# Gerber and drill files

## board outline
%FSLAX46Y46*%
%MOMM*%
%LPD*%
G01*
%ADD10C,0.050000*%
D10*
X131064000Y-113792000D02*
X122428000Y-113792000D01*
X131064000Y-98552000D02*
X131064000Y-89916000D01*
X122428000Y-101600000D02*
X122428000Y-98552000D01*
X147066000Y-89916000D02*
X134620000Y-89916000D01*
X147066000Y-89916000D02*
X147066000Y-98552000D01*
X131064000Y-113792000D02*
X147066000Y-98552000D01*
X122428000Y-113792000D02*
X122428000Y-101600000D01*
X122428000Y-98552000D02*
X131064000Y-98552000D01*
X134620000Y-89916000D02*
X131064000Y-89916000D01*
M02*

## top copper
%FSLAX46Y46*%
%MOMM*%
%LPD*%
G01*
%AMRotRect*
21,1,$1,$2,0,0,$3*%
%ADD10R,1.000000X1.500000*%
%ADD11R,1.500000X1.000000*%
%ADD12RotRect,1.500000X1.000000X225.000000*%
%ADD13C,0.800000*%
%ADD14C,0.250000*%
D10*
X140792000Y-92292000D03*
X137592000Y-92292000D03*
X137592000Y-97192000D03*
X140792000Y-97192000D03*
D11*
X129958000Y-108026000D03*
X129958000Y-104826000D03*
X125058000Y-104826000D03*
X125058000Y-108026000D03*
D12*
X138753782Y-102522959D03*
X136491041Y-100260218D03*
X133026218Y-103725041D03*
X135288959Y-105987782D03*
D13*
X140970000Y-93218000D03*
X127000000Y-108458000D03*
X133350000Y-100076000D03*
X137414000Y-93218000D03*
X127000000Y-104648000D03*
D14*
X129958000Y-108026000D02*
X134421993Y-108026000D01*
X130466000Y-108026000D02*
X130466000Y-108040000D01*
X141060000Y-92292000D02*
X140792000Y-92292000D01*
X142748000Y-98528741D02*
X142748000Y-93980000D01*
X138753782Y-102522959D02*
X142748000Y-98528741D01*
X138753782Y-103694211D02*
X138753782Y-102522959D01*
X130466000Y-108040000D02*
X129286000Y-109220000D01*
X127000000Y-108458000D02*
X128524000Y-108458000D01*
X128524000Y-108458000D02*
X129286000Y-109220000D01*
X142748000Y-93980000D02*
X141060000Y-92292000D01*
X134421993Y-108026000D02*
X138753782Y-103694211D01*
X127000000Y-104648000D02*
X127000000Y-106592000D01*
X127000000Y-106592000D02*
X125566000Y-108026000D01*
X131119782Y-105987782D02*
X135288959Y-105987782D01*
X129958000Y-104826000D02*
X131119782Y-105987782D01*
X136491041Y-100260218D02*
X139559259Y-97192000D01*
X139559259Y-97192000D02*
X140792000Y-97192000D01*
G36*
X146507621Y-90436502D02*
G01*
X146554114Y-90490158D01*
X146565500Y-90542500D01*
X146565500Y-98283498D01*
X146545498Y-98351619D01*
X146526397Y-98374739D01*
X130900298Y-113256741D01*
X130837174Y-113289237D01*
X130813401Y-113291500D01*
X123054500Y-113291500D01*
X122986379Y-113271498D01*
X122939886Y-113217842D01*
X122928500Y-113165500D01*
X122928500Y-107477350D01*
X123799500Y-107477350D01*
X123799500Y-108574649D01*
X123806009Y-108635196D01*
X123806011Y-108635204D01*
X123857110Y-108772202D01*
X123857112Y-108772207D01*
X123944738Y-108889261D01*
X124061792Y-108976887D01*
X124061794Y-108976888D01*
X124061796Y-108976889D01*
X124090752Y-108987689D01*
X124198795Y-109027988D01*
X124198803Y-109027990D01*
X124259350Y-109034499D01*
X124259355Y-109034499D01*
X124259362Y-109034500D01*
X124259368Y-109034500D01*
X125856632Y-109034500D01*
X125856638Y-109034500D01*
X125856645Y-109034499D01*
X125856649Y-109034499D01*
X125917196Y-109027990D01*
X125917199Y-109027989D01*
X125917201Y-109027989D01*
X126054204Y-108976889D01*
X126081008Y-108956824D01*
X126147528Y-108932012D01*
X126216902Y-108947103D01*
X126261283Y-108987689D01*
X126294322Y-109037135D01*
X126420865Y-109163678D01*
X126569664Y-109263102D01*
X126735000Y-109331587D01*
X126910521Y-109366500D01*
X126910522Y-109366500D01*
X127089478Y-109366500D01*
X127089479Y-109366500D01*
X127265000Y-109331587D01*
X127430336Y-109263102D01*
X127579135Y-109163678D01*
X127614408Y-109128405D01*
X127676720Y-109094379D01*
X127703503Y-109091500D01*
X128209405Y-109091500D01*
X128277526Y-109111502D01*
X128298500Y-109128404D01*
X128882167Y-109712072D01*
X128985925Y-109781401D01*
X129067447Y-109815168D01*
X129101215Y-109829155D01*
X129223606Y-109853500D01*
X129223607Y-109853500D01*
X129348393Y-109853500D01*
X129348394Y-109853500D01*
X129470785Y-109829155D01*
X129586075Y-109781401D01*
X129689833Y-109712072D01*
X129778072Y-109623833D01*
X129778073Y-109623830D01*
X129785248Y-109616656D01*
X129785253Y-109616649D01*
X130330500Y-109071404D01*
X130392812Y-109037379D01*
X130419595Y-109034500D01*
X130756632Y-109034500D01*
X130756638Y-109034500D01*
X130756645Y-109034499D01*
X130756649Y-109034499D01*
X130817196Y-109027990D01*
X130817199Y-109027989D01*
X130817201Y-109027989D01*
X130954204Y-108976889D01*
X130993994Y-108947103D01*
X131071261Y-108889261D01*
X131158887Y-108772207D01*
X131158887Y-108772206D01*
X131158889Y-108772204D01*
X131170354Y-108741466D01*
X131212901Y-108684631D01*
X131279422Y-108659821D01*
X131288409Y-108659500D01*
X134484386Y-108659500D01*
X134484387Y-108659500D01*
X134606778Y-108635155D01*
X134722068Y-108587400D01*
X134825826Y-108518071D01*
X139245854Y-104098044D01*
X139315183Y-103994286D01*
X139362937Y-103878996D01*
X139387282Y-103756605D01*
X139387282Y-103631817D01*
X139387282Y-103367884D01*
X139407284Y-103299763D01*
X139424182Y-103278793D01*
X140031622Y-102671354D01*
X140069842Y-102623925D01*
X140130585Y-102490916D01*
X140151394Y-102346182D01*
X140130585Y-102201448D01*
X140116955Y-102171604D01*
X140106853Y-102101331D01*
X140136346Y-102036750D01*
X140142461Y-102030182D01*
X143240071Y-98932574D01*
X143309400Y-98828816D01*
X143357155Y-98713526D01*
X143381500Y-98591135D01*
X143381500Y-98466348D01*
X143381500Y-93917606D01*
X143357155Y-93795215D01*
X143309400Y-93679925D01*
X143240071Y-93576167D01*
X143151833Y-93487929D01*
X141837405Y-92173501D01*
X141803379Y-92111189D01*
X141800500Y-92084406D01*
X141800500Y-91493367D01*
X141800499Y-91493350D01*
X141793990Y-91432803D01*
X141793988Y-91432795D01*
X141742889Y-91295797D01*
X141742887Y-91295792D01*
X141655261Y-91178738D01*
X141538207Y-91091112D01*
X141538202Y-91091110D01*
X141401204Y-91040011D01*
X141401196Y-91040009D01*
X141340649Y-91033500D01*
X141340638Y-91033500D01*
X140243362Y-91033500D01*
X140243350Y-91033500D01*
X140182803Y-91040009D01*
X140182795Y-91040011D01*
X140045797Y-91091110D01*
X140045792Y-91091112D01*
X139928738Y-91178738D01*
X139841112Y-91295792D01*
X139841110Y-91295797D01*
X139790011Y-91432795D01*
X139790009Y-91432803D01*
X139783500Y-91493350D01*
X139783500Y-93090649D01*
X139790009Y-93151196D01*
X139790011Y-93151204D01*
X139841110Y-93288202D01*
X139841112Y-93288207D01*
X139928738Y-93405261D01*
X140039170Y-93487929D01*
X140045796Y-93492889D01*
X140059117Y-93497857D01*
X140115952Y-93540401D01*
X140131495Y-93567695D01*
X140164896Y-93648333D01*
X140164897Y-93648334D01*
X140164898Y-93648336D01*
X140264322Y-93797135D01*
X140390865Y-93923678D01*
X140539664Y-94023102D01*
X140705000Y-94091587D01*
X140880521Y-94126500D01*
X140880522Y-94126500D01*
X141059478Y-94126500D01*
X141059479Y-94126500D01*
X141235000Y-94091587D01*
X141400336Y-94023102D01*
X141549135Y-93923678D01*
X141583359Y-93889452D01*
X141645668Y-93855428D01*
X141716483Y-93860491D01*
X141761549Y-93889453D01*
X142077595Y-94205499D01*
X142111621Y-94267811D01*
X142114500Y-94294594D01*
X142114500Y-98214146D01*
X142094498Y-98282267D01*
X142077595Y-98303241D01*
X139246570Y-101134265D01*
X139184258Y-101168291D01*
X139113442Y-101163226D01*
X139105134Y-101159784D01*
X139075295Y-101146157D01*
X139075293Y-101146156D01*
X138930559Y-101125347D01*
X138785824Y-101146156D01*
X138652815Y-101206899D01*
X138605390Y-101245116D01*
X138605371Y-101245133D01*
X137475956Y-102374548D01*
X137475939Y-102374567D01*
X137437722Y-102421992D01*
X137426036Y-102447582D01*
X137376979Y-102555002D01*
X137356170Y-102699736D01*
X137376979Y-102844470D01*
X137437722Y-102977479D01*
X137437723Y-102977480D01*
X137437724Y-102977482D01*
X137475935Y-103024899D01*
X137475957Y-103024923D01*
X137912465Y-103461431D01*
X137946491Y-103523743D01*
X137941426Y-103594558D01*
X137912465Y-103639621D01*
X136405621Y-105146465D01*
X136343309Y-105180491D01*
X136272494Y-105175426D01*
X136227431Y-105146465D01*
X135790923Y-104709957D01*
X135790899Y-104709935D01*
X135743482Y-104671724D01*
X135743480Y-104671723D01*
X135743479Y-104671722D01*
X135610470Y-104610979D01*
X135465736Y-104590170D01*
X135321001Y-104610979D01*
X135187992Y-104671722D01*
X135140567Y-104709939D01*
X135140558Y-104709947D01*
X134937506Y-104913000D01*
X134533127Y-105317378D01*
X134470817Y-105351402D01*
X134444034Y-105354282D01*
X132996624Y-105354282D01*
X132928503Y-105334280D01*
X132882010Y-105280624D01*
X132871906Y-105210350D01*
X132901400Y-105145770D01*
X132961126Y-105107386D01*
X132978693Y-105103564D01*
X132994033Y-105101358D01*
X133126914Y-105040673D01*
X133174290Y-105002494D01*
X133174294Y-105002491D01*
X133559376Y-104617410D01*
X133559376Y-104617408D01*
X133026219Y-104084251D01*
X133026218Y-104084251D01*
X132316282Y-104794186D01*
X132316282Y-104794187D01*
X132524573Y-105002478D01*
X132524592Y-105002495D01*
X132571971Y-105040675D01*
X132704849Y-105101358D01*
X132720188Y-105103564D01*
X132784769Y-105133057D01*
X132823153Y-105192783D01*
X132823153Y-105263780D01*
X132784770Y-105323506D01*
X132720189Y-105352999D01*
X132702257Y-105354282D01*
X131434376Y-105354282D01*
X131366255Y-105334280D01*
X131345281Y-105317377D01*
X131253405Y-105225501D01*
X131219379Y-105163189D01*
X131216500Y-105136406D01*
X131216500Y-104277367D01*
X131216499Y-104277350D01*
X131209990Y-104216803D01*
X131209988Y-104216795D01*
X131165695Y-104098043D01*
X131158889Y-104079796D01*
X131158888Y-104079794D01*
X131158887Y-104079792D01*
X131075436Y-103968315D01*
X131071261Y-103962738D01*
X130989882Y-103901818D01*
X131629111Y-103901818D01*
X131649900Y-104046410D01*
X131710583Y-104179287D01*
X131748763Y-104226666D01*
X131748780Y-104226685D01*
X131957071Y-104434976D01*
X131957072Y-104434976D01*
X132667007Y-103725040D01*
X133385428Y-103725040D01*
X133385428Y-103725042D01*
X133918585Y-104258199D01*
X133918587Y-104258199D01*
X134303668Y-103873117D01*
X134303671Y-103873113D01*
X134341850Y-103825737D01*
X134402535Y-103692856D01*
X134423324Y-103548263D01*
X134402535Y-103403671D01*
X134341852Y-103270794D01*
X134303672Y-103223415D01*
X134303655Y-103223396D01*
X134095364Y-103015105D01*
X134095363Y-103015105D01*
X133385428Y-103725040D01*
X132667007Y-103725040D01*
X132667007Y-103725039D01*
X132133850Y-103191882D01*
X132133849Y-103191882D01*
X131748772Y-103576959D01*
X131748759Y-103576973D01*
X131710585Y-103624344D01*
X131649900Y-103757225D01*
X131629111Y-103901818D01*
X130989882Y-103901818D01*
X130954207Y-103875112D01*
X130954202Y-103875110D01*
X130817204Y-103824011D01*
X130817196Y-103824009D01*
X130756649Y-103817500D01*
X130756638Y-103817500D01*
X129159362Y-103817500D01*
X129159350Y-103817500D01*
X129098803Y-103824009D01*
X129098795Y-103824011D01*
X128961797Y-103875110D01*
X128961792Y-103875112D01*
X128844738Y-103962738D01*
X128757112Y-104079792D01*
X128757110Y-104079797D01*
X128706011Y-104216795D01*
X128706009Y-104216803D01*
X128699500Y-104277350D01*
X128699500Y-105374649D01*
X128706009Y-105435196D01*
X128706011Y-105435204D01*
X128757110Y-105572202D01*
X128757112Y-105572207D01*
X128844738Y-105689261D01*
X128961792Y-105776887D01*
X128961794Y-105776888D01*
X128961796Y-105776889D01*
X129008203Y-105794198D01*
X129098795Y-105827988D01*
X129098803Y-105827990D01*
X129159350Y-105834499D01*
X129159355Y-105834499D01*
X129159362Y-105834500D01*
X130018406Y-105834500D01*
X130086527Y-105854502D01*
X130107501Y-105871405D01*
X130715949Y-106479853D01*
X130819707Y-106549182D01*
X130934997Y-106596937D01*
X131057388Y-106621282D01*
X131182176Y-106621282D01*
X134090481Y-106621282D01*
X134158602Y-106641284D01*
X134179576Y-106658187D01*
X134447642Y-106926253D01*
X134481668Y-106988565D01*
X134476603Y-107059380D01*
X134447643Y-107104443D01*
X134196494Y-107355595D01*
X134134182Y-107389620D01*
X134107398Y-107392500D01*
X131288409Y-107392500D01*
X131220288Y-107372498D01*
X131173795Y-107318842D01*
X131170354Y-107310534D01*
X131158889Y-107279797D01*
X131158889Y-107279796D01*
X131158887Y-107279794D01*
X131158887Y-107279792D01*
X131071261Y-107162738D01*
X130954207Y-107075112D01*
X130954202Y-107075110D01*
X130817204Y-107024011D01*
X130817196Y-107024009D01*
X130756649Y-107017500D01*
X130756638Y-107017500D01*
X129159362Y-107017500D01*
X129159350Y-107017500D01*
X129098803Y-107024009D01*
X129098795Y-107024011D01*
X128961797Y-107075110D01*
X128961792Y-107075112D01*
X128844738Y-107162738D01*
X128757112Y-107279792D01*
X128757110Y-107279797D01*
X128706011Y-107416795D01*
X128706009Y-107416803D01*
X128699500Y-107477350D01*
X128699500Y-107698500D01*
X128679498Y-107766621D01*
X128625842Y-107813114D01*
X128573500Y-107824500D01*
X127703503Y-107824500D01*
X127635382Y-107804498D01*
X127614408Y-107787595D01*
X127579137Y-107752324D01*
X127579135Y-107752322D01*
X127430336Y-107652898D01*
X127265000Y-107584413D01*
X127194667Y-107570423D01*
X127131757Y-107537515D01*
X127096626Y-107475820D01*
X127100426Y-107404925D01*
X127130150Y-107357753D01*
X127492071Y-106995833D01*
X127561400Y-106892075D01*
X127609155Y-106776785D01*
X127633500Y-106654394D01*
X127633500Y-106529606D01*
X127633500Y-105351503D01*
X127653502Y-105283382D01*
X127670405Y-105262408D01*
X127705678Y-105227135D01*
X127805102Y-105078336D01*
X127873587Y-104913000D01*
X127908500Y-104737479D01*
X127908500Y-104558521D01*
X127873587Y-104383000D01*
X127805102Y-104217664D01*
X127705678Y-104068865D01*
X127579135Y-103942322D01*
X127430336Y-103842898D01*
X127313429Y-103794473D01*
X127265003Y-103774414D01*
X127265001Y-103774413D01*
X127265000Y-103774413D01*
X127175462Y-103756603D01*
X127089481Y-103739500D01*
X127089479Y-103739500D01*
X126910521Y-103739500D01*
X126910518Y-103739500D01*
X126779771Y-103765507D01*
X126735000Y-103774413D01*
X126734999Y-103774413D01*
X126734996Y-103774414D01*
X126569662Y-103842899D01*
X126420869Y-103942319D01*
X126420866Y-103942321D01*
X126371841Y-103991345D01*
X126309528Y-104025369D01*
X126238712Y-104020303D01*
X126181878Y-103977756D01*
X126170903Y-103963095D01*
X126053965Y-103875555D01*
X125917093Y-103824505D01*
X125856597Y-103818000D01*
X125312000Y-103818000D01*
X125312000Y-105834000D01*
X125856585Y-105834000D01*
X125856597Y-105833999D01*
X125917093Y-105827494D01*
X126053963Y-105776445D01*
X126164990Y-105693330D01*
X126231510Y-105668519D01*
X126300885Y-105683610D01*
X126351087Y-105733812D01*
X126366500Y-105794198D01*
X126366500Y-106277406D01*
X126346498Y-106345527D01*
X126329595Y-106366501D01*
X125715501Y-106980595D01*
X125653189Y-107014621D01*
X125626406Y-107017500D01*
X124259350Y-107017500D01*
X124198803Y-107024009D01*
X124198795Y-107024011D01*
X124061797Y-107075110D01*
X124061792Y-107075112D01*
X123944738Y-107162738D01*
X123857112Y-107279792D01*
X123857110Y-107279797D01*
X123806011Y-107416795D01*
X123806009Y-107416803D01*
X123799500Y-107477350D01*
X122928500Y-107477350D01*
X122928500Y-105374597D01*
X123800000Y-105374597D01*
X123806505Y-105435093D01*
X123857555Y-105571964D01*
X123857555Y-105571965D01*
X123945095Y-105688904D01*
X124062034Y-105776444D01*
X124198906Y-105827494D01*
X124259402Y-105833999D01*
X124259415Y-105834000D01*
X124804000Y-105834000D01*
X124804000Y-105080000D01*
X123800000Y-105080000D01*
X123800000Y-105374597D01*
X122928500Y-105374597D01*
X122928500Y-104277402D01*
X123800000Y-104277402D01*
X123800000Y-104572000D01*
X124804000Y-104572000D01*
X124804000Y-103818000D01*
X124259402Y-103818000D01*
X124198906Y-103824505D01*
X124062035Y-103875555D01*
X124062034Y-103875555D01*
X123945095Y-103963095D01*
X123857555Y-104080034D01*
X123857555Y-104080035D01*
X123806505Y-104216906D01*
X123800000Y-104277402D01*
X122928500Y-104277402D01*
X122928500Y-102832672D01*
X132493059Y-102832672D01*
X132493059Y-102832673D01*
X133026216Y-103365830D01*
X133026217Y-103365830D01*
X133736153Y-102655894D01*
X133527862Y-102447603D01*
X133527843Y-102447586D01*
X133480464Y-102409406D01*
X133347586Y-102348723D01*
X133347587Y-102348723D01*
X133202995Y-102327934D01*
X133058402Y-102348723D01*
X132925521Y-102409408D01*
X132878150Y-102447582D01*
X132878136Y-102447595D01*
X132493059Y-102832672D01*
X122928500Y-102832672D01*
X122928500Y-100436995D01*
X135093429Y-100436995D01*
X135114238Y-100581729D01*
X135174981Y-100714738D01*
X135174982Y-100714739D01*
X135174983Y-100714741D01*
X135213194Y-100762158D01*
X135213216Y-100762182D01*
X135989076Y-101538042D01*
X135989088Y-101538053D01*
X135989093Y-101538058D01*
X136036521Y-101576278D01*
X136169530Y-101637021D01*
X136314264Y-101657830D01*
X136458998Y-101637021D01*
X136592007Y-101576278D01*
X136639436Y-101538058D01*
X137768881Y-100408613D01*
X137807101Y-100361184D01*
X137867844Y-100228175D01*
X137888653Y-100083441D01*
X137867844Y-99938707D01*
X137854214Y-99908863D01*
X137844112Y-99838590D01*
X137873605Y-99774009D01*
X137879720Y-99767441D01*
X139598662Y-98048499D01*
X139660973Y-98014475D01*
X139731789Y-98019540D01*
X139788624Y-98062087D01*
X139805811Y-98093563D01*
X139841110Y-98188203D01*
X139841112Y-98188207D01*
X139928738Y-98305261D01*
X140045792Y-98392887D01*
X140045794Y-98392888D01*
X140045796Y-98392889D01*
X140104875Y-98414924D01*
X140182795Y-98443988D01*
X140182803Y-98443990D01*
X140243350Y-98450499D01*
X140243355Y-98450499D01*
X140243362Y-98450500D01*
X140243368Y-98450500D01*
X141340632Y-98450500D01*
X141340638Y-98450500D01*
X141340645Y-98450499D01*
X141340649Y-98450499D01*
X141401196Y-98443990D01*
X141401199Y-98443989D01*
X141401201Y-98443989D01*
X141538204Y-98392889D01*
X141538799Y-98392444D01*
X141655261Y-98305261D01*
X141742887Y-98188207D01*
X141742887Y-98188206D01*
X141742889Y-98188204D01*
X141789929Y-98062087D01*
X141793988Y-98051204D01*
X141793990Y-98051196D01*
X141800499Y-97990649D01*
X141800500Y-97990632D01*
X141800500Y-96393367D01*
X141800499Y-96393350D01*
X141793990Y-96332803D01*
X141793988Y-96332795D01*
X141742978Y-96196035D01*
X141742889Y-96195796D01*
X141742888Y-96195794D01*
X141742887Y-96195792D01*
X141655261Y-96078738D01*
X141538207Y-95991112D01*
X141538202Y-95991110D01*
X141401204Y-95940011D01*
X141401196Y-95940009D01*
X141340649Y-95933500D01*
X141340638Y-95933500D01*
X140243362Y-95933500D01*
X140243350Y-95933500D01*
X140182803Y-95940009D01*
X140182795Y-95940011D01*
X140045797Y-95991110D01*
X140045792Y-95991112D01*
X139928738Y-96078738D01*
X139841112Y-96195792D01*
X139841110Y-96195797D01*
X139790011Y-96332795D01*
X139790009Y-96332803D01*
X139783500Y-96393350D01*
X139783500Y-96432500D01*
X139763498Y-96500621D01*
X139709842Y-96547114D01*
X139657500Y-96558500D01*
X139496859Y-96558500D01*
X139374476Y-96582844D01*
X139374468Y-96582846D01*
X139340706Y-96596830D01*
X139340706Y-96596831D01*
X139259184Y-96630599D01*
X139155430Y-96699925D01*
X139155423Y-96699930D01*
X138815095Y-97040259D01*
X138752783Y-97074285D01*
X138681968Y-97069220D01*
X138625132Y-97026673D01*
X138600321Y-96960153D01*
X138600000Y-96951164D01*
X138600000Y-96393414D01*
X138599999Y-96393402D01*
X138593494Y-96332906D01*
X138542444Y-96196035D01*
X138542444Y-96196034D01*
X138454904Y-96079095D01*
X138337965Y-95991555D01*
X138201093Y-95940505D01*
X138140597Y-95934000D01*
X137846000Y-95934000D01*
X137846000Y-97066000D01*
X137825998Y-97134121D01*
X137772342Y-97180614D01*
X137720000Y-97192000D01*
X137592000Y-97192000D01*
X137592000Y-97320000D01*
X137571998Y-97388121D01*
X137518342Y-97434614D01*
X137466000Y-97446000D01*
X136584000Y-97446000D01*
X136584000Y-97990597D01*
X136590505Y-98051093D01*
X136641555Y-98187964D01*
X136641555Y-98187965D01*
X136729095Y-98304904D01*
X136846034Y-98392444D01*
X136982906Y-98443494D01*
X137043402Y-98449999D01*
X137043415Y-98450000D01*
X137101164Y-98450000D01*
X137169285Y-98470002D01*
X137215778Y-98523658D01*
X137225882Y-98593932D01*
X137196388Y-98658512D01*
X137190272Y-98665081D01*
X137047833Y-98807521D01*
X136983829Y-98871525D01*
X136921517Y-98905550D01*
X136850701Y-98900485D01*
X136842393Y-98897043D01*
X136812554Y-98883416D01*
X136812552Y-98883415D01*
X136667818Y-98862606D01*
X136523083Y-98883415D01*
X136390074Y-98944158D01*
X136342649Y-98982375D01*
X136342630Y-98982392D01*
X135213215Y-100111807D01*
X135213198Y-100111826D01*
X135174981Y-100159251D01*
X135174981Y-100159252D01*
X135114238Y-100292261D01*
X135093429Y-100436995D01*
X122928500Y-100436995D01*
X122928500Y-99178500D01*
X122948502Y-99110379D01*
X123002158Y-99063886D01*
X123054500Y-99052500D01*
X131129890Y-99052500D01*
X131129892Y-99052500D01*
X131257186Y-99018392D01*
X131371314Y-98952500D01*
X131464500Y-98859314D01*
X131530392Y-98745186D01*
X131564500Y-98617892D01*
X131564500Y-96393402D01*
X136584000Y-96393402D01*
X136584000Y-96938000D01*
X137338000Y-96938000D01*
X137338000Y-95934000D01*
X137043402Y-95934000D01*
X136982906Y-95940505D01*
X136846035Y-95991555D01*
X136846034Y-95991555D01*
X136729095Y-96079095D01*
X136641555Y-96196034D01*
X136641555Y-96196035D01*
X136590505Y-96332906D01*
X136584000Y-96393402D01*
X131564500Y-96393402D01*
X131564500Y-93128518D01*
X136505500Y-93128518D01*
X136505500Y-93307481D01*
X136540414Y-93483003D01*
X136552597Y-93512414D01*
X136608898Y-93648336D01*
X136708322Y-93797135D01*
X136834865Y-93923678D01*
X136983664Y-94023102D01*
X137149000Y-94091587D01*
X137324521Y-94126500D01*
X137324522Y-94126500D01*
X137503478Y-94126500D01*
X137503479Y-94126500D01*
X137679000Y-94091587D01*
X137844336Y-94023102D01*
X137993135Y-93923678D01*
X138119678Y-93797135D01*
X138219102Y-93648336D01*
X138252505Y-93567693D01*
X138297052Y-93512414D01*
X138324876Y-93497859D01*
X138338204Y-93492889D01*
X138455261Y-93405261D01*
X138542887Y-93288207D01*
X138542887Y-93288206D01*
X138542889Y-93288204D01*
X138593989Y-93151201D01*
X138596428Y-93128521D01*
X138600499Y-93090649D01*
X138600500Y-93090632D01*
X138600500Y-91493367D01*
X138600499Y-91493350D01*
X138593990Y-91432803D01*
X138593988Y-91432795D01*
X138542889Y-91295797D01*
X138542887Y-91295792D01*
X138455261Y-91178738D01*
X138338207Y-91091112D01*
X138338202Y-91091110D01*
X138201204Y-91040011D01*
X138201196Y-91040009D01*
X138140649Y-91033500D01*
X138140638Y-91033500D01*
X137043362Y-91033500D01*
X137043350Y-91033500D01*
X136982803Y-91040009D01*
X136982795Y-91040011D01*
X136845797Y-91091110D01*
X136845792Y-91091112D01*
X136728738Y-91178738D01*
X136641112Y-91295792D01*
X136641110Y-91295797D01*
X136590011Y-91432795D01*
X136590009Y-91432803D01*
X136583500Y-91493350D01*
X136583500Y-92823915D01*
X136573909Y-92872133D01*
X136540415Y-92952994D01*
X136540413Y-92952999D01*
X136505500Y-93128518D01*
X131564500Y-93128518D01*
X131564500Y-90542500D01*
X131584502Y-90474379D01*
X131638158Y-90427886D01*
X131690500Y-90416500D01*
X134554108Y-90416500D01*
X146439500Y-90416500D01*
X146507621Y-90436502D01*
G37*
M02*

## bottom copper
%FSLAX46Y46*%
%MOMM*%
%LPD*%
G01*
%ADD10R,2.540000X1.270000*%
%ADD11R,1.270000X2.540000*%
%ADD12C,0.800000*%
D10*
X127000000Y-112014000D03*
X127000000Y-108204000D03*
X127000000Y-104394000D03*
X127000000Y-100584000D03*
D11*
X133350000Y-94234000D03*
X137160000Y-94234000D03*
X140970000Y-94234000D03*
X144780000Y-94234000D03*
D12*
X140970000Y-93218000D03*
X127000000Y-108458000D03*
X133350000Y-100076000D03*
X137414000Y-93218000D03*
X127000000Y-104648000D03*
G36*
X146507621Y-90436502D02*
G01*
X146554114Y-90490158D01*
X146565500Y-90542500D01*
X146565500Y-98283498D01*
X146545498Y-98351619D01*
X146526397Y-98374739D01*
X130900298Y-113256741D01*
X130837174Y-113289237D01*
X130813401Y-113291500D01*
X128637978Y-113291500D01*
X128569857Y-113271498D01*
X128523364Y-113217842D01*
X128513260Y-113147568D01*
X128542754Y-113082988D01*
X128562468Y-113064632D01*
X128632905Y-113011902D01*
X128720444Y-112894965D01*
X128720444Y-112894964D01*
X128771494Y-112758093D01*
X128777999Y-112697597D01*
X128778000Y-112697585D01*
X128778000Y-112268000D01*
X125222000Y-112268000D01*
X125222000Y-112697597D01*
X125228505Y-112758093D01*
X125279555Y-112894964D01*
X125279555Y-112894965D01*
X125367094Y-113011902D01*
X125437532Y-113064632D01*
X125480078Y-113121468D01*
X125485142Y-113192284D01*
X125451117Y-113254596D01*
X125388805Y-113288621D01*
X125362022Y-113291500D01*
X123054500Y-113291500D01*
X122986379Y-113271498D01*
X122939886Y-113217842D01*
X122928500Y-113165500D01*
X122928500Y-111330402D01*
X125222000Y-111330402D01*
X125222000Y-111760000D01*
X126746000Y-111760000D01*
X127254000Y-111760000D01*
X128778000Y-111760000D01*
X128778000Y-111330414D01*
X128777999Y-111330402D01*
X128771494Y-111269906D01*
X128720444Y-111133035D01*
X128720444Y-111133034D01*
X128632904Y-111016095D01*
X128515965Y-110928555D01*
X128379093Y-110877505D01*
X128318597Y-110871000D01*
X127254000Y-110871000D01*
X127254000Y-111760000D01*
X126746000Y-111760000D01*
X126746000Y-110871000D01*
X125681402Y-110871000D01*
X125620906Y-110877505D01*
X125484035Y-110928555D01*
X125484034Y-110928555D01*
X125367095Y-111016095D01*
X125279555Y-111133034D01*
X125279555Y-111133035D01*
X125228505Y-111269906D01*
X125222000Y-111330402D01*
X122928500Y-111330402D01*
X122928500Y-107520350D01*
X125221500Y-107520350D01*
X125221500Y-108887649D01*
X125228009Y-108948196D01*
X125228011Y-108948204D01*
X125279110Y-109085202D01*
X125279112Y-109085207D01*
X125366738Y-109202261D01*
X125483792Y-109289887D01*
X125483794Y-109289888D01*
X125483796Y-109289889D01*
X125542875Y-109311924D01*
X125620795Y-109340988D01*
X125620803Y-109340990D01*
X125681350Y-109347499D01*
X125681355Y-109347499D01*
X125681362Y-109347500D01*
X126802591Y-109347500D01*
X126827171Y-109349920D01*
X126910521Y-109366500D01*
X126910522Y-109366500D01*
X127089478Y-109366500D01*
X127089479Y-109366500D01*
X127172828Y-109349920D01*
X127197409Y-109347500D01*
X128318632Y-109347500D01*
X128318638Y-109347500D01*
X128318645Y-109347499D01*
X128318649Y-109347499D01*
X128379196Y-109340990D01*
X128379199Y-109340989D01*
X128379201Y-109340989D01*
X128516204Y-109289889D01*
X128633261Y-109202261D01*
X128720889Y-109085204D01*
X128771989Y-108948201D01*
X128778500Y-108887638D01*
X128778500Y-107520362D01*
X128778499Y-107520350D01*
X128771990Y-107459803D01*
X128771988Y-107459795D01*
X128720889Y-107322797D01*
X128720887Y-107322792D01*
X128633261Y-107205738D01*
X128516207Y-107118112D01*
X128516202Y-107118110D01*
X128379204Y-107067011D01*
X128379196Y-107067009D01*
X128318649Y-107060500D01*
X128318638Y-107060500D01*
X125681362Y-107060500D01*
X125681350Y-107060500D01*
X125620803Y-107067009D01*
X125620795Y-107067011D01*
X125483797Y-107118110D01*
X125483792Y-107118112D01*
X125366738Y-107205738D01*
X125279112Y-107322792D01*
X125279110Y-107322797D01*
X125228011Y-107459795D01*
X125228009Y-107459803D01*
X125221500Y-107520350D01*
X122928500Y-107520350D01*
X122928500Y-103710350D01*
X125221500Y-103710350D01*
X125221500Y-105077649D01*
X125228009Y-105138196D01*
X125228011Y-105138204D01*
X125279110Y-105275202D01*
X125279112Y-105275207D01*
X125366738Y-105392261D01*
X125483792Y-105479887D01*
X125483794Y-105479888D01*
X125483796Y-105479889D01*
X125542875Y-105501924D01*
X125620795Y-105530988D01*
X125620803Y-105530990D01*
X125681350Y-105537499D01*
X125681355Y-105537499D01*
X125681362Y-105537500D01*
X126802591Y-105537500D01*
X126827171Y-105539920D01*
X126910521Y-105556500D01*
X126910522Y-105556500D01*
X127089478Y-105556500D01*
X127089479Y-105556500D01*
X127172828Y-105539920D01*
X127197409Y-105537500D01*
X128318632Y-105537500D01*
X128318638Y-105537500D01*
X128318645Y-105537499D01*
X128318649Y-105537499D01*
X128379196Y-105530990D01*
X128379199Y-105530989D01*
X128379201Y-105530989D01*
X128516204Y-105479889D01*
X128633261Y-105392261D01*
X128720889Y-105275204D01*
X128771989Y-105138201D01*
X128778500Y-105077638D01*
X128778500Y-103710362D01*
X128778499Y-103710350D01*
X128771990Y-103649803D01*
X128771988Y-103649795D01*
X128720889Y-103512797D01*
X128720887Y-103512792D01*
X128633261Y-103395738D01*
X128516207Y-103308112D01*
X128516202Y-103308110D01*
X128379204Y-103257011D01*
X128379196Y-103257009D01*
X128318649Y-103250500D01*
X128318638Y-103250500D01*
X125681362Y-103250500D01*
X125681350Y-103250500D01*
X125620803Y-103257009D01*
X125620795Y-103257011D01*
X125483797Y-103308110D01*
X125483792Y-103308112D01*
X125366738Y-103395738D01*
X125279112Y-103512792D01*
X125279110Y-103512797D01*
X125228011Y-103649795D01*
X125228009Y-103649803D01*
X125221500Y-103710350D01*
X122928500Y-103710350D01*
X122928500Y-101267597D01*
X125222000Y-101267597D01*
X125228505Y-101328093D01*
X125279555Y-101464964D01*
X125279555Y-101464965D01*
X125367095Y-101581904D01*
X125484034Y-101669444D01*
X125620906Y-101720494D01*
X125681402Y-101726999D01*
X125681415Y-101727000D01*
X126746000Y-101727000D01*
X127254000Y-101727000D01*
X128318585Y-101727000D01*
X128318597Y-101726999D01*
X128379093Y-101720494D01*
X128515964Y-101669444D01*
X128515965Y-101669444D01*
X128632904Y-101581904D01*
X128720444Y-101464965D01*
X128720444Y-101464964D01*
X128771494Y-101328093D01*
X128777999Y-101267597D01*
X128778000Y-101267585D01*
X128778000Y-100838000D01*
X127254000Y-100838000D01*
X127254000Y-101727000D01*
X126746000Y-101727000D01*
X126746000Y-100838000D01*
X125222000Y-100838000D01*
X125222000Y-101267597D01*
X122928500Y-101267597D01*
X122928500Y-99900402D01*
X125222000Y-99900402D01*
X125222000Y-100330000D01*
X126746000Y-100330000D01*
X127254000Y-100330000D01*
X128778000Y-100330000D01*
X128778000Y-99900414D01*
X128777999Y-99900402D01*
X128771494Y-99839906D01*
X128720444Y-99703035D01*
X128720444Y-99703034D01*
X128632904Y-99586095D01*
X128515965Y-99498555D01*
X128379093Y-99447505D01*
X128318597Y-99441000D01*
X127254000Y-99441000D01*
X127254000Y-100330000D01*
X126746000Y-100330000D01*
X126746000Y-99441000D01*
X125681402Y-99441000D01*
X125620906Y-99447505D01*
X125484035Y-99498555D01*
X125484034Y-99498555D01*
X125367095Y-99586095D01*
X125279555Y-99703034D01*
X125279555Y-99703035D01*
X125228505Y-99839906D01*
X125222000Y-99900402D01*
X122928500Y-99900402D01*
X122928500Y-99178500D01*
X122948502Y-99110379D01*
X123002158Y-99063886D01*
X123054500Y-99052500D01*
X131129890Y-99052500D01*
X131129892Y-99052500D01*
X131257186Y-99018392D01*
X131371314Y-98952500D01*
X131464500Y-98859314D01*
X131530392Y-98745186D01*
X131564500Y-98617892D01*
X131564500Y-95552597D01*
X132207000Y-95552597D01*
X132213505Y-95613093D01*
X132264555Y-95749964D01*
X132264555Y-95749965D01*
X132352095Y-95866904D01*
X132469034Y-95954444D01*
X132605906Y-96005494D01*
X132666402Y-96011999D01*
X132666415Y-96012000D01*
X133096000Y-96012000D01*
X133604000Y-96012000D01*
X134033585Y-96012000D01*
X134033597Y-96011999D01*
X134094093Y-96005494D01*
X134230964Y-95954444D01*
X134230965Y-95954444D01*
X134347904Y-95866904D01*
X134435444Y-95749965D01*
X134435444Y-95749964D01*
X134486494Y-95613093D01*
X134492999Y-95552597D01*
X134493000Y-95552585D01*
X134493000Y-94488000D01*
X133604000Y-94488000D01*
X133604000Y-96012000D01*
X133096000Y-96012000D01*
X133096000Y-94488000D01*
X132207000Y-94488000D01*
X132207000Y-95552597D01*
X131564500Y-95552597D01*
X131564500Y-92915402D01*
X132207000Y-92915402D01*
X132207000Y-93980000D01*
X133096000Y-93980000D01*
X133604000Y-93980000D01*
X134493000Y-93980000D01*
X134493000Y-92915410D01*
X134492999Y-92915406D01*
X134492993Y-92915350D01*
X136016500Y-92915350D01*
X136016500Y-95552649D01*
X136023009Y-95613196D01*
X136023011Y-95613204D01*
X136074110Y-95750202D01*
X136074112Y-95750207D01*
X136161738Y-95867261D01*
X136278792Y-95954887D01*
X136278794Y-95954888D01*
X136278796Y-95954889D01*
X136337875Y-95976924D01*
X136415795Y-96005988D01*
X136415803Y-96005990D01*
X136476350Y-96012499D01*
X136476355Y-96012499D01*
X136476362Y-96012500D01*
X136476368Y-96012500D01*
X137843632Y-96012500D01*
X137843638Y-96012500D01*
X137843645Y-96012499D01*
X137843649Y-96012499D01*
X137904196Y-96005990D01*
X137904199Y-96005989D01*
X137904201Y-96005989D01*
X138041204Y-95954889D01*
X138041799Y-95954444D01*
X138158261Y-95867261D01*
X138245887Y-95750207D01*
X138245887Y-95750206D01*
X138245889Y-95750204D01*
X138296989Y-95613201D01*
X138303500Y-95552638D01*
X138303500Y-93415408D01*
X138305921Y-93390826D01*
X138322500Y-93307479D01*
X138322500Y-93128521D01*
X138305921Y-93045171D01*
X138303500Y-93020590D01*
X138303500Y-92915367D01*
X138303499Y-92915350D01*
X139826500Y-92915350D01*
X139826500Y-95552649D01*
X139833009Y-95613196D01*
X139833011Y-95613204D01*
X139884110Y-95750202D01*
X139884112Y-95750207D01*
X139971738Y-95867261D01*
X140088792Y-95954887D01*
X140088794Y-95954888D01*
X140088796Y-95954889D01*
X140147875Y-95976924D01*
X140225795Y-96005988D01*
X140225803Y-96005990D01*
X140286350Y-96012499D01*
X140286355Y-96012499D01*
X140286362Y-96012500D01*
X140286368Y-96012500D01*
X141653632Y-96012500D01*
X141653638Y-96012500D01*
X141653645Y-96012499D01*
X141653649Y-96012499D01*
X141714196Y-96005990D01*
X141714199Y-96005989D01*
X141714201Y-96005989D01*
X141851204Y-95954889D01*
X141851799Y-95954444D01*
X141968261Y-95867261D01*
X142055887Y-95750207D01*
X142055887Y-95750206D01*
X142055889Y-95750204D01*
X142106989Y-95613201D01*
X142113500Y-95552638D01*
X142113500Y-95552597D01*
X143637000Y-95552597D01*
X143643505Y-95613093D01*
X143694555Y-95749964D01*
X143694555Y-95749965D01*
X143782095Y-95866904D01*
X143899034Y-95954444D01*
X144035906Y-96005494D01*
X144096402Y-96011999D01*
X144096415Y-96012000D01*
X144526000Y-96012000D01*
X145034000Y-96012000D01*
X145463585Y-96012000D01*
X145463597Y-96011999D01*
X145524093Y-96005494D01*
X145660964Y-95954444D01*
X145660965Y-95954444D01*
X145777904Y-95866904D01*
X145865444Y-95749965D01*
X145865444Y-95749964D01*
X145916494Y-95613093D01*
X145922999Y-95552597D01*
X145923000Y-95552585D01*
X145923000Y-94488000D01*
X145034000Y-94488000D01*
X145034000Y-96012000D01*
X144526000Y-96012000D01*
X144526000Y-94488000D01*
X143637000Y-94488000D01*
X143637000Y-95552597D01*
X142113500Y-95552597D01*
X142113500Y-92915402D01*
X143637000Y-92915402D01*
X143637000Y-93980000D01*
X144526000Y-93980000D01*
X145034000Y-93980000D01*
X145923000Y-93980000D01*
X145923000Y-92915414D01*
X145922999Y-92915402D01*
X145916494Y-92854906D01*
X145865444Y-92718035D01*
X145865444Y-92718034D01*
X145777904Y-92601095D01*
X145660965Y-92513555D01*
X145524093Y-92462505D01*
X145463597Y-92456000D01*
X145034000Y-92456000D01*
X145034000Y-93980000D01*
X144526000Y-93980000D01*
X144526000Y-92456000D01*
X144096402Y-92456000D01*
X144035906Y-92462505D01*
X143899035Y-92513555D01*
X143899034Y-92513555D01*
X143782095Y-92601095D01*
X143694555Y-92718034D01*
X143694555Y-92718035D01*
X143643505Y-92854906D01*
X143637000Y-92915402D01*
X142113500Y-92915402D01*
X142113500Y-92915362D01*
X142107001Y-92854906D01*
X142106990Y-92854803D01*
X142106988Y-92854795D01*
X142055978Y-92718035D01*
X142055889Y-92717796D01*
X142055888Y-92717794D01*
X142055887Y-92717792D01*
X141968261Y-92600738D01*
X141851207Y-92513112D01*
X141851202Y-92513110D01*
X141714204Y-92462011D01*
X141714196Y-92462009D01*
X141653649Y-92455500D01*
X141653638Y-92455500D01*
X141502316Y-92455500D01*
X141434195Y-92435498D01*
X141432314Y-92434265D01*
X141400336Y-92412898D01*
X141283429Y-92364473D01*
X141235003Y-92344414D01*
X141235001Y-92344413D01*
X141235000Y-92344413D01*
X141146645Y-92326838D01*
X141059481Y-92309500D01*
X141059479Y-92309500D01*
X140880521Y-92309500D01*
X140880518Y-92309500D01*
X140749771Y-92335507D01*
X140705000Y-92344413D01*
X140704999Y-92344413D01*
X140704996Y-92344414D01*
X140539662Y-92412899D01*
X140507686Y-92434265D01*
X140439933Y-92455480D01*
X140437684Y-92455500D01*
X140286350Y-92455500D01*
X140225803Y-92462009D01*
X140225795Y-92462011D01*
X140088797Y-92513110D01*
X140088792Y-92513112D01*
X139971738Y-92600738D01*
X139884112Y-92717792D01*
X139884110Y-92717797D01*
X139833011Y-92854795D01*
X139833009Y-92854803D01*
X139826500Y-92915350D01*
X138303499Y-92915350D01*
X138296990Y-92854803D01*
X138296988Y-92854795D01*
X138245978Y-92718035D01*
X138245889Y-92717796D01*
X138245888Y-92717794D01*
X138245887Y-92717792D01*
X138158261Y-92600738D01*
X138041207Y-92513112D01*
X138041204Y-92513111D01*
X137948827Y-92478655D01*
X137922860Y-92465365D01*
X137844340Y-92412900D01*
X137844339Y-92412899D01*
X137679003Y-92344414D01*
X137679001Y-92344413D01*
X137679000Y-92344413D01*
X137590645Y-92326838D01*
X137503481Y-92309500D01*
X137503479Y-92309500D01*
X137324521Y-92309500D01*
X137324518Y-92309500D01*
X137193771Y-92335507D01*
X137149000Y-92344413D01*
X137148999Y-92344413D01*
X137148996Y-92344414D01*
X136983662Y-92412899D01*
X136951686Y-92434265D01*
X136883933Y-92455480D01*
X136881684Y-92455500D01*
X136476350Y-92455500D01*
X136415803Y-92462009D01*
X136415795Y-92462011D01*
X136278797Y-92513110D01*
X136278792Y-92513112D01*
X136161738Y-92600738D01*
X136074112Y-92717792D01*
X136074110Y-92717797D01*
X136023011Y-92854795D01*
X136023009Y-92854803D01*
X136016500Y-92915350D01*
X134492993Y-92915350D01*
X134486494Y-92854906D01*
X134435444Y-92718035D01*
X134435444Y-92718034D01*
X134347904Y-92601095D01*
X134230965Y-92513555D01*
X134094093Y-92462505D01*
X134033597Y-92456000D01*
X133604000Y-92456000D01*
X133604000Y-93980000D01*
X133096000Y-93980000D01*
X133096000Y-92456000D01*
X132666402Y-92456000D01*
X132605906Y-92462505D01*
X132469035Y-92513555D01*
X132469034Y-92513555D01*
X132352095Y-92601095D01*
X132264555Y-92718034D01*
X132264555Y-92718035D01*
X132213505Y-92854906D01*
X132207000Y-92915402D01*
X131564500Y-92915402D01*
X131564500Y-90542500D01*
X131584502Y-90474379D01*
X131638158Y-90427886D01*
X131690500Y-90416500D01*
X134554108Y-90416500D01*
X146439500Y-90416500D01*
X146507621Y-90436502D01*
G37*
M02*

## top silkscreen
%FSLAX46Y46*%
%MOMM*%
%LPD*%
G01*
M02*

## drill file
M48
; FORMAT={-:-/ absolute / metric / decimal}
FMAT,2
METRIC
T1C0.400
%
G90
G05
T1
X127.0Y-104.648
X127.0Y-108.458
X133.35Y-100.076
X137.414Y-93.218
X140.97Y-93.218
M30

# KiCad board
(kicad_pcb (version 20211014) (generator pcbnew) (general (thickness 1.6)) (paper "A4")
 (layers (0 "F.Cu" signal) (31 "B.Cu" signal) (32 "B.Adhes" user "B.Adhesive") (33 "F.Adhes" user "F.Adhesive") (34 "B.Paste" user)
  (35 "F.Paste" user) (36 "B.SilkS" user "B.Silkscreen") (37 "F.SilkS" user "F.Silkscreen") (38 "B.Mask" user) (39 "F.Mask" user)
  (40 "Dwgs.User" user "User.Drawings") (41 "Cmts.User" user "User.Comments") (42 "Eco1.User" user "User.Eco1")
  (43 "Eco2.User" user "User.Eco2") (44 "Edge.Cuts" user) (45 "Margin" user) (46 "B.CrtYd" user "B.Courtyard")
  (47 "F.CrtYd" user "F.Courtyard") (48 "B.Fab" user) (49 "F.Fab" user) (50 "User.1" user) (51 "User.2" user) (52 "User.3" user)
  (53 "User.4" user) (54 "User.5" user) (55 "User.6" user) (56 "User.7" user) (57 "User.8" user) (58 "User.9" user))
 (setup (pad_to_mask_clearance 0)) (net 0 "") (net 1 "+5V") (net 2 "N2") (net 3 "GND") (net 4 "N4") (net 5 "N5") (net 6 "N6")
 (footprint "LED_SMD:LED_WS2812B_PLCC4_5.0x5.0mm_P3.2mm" (layer "F.Cu") (at 139.192 94.742 -90)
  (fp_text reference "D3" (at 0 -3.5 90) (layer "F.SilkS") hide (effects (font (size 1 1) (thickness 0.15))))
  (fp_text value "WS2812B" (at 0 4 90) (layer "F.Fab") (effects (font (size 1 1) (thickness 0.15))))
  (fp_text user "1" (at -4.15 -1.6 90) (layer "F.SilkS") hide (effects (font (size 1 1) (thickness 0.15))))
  (pad "1" smd rect (at -2.45 -1.6 270) (size 1.5 1) (layers "F.Cu" "F.Paste" "F.Mask") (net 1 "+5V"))
  (pad "2" smd rect (at -2.45 1.6 270) (size 1.5 1) (layers "F.Cu" "F.Paste" "F.Mask") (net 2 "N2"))
  (pad "3" smd rect (at 2.45 1.6 270) (size 1.5 1) (layers "F.Cu" "F.Paste" "F.Mask") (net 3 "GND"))
  (pad "4" smd rect (at 2.45 -1.6 270) (size 1.5 1) (layers "F.Cu" "F.Paste" "F.Mask") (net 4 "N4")))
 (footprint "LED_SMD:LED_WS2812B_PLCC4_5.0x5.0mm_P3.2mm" (layer "F.Cu") (at 127.508 106.426 180)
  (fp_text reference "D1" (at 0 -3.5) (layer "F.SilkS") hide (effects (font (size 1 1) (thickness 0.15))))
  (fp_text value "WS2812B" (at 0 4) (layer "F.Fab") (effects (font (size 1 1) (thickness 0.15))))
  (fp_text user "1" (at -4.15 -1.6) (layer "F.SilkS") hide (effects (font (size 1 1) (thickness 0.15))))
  (pad "1" smd rect (at -2.45 -1.6 180) (size 1.5 1) (layers "F.Cu" "F.Paste" "F.Mask") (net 1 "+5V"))
  (pad "2" smd rect (at -2.45 1.6 180) (size 1.5 1) (layers "F.Cu" "F.Paste" "F.Mask") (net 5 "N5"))
  (pad "3" smd rect (at 2.45 1.6 180) (size 1.5 1) (layers "F.Cu" "F.Paste" "F.Mask") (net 3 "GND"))
  (pad "4" smd rect (at 2.45 -1.6 180) (size 1.5 1) (layers "F.Cu" "F.Paste" "F.Mask") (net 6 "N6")))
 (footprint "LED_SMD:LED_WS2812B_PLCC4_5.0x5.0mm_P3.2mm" (layer "F.Cu") (at 135.89 103.124 -135)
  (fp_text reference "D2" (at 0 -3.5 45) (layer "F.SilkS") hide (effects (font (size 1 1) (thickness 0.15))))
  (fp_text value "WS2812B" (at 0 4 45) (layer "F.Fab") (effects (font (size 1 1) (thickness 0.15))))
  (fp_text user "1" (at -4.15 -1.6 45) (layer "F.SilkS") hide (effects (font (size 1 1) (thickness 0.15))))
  (pad "1" smd rect (at -2.45 -1.6 225) (size 1.5 1) (layers "F.Cu" "F.Paste" "F.Mask") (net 1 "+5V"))
  (pad "2" smd rect (at -2.45 1.6 225) (size 1.5 1) (layers "F.Cu" "F.Paste" "F.Mask") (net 4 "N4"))
  (pad "3" smd rect (at 2.45 1.6 225) (size 1.5 1) (layers "F.Cu" "F.Paste" "F.Mask") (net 3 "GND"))
  (pad "4" smd rect (at 2.45 -1.6 225) (size 1.5 1) (layers "F.Cu" "F.Paste" "F.Mask") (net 5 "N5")))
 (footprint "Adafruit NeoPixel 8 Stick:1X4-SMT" (layer "B.Cu") (at 127 106.934 90)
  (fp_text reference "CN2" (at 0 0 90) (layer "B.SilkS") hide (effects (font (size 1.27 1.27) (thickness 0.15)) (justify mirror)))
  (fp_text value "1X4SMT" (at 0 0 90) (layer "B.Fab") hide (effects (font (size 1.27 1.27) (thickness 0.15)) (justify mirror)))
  (pad "1" smd rect (at -5.08 0 90) (size 1.27 2.54) (layers "B.Cu" "B.Paste" "B.Mask") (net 3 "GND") (solder_mask_margin 0.1016))
  (pad "2" smd rect (at -1.27 0 90) (size 1.27 2.54) (layers "B.Cu" "B.Paste" "B.Mask") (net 1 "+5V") (solder_mask_margin 0.1016))
  (pad "3" smd rect (at 2.54 0 90) (size 1.27 2.54) (layers "B.Cu" "B.Paste" "B.Mask") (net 6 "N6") (solder_mask_margin 0.1016))
  (pad "4" smd rect (at 6.35 0 90) (size 1.27 2.54) (layers "B.Cu" "B.Paste" "B.Mask") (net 3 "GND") (solder_mask_margin 0.1016)))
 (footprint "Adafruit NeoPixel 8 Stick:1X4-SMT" (layer "B.Cu") (at 138.43 94.234)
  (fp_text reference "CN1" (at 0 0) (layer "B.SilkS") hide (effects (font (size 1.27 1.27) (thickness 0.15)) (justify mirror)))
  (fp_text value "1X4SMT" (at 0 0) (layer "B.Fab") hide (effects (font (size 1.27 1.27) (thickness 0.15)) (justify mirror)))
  (pad "1" smd rect (at -5.08 0) (size 1.27 2.54) (layers "B.Cu" "B.Paste" "B.Mask") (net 3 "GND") (solder_mask_margin 0.1016))
  (pad "2" smd rect (at -1.27 0) (size 1.27 2.54) (layers "B.Cu" "B.Paste" "B.Mask") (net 2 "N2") (solder_mask_margin 0.1016))
  (pad "3" smd rect (at 2.54 0) (size 1.27 2.54) (layers "B.Cu" "B.Paste" "B.Mask") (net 1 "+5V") (solder_mask_margin 0.1016))
  (pad "4" smd rect (at 6.35 0) (size 1.27 2.54) (layers "B.Cu" "B.Paste" "B.Mask") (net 3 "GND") (solder_mask_margin 0.1016)))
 (gr_line (start 131.064 113.792) (end 122.428 113.792) (layer "Edge.Cuts") (width 0.05))
 (gr_line (start 131.064 98.552) (end 131.064 89.916) (layer "Edge.Cuts") (width 0.05))
 (gr_line (start 122.428 101.6) (end 122.428 98.552) (layer "Edge.Cuts") (width 0.05))
 (gr_line (start 147.066 89.916) (end 134.62 89.916) (layer "Edge.Cuts") (width 0.05))
 (gr_line (start 147.066 89.916) (end 147.066 98.552) (layer "Edge.Cuts") (width 0.05))
 (gr_line (start 131.064 113.792) (end 147.066 98.552) (layer "Edge.Cuts") (width 0.05))
 (gr_line (start 122.428 113.792) (end 122.428 101.6) (layer "Edge.Cuts") (width 0.05))
 (gr_line (start 122.428 98.552) (end 131.064 98.552) (layer "Edge.Cuts") (width 0.05))
 (gr_line (start 134.62 89.916) (end 131.064 89.916) (layer "Edge.Cuts") (width 0.05))
 (segment (start 129.958 108.026) (end 134.421993 108.026) (width 0.25) (layer "F.Cu") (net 1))
 (segment (start 130.466 108.026) (end 130.466 108.04) (width 0.25) (layer "F.Cu") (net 1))
 (segment (start 141.06 92.292) (end 140.792 92.292) (width 0.25) (layer "F.Cu") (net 1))
 (segment (start 142.748 98.528741) (end 142.748 93.98) (width 0.25) (layer "F.Cu") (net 1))
 (segment (start 138.753782 102.522959) (end 142.748 98.528741) (width 0.25) (layer "F.Cu") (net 1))
 (segment (start 138.753782 103.694211) (end 138.753782 102.522959) (width 0.25) (layer "F.Cu") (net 1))
 (segment (start 130.466 108.04) (end 129.286 109.22) (width 0.25) (layer "F.Cu") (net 1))
 (segment (start 127 108.458) (end 128.524 108.458) (width 0.25) (layer "F.Cu") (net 1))
 (segment (start 128.524 108.458) (end 129.286 109.22) (width 0.25) (layer "F.Cu") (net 1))
 (segment (start 142.748 93.98) (end 141.06 92.292) (width 0.25) (layer "F.Cu") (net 1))
 (segment (start 134.421993 108.026) (end 138.753782 103.694211) (width 0.25) (layer "F.Cu") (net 1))
 (via (at 140.97 93.218) (size 0.8) (drill 0.4) (layers "F.Cu" "B.Cu") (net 1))
 (via (at 127 108.458) (size 0.8) (drill 0.4) (layers "F.Cu" "B.Cu") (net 1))
 (via (at 133.35 100.076) (size 0.8) (drill 0.4) (layers "F.Cu" "B.Cu") (free) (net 3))
 (via (at 137.414 93.218) (size 0.8) (drill 0.4) (layers "F.Cu" "B.Cu") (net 2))
 (segment (start 127 104.648) (end 127 106.592) (width 0.25) (layer "F.Cu") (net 6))
 (segment (start 127 106.592) (end 125.566 108.026) (width 0.25) (layer "F.Cu") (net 6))
 (via (at 127 104.648) (size 0.8) (drill 0.4) (layers "F.Cu" "B.Cu") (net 6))
 (segment (start 131.119782 105.987782) (end 135.288959 105.987782) (width 0.25) (layer "F.Cu") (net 5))
 (segment (start 129.958 104.826) (end 131.119782 105.987782) (width 0.25) (layer "F.Cu") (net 5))
 (segment (start 136.491041 100.260218) (end 139.559259 97.192) (width 0.25) (layer "F.Cu") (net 4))
 (segment (start 139.559259 97.192) (end 140.792 97.192) (width 0.25) (layer "F.Cu") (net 4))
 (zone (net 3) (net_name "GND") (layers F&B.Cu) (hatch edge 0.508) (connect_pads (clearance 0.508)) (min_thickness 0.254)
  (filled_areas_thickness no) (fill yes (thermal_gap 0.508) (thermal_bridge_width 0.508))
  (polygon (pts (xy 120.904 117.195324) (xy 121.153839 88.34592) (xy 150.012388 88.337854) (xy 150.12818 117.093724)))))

